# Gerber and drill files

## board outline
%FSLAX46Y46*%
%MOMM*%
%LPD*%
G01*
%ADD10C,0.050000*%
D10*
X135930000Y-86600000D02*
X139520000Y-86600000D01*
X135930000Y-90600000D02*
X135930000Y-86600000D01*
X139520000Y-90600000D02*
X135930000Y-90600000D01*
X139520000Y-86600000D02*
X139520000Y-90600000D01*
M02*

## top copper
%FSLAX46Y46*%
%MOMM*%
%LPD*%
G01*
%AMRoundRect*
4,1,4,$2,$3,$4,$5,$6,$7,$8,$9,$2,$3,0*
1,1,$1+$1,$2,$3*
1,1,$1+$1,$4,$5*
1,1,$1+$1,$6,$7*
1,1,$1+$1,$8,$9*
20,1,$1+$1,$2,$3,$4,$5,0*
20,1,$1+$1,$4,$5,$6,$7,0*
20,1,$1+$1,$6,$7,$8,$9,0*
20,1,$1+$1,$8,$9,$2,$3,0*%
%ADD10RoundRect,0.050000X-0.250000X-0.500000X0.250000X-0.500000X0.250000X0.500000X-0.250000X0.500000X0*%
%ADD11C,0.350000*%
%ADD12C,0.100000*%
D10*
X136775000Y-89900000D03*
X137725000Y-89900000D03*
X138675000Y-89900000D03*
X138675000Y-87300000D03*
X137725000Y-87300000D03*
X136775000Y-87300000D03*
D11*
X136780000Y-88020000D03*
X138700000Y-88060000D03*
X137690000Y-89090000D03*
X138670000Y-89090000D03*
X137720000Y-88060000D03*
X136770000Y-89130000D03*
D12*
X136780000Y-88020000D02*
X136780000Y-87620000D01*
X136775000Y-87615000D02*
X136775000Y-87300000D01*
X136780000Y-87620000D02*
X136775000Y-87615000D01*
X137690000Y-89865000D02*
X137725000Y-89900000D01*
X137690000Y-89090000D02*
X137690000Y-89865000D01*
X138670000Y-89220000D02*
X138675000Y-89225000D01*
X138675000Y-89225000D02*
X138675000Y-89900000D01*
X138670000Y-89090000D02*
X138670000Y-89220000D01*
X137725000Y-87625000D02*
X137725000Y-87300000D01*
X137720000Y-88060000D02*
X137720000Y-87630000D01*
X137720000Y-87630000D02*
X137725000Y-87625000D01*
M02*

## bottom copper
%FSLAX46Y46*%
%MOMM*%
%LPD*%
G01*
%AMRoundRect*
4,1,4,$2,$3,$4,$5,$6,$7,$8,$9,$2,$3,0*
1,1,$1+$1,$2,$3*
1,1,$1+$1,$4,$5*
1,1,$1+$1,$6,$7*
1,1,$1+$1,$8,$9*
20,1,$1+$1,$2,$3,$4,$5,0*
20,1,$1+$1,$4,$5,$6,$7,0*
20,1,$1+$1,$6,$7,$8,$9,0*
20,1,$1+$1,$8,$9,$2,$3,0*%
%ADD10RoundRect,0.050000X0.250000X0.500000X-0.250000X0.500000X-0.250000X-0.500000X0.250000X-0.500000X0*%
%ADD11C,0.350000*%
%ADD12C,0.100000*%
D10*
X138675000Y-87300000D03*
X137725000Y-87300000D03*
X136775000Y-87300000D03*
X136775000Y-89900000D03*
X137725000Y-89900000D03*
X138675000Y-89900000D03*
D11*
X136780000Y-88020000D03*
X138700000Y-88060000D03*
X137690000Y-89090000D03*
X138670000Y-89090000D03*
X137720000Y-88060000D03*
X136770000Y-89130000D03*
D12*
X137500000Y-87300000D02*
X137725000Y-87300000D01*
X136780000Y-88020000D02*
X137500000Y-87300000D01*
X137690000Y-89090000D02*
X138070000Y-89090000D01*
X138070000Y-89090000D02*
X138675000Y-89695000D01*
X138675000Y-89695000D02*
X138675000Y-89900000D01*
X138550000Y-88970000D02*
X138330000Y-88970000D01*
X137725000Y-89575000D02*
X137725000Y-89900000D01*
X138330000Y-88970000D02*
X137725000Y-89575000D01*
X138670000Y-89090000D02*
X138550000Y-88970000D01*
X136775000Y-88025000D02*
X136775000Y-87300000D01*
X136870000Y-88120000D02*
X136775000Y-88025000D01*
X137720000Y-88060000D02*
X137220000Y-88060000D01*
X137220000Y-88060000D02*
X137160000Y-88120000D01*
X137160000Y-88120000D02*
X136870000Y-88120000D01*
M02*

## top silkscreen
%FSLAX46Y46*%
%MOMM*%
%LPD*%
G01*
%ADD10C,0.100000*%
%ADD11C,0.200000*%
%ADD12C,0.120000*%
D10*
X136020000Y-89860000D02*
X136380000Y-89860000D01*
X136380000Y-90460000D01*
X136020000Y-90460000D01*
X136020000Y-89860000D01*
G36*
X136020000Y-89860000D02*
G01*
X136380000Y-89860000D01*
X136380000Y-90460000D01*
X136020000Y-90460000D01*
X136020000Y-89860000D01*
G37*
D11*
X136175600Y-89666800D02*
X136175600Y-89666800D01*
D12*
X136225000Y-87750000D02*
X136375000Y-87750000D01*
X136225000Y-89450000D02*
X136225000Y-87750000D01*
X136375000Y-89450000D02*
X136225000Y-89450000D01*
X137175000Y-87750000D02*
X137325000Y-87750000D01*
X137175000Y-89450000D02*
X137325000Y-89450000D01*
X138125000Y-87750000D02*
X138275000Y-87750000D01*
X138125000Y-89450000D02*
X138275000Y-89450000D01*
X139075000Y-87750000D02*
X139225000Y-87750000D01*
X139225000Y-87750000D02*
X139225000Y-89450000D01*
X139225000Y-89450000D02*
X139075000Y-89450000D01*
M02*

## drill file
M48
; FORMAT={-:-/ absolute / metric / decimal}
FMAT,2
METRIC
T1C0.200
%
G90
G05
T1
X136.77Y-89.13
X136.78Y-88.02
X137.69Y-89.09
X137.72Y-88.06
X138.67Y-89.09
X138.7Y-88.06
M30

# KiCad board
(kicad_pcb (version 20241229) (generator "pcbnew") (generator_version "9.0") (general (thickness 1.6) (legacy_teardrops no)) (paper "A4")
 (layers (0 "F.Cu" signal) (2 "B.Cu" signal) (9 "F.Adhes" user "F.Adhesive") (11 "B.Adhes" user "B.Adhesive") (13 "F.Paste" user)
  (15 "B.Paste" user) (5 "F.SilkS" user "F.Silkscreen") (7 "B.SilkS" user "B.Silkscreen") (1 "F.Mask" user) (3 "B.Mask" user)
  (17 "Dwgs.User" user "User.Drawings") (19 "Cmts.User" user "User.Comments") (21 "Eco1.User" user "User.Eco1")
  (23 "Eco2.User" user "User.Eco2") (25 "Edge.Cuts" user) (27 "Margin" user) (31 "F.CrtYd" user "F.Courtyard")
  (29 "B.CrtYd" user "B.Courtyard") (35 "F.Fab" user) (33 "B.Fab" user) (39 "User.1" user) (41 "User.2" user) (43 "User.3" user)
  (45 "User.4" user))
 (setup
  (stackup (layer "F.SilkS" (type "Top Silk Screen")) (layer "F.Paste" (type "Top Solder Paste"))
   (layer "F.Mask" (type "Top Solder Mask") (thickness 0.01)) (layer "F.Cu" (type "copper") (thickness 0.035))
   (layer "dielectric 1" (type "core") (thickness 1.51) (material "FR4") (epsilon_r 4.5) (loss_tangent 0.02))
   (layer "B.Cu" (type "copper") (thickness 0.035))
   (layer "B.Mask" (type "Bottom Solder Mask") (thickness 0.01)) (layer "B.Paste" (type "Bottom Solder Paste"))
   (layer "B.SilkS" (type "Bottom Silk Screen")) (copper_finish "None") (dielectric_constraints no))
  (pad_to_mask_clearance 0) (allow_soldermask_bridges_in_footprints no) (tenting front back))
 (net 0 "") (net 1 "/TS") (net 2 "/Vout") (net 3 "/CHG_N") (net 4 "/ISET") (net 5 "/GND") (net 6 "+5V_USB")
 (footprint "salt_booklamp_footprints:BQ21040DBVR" (layer "F.Cu") (at 137.725 88.6)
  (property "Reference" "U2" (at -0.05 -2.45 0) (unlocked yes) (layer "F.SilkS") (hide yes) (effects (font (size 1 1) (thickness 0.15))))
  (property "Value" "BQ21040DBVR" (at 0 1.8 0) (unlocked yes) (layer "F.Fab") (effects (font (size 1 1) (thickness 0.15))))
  (fp_line (start -1.5494 1.0668) (end -1.5494 1.0668) (stroke (width 0.2) (type default)) (layer "F.SilkS"))
  (fp_line (start -1.5 -0.85) (end -1.35 -0.85) (stroke (width 0.12) (type default)) (layer "F.SilkS"))
  (fp_line (start -1.5 0.85) (end -1.5 -0.85) (stroke (width 0.12) (type default)) (layer "F.SilkS"))
  (fp_line (start -1.35 0.85) (end -1.5 0.85) (stroke (width 0.12) (type default)) (layer "F.SilkS"))
  (fp_line (start -0.55 -0.85) (end -0.4 -0.85) (stroke (width 0.12) (type default)) (layer "F.SilkS"))
  (fp_line (start -0.55 0.85) (end -0.4 0.85) (stroke (width 0.12) (type default)) (layer "F.SilkS"))
  (fp_line (start 0.4 -0.85) (end 0.55 -0.85) (stroke (width 0.12) (type default)) (layer "F.SilkS"))
  (fp_line (start 0.4 0.85) (end 0.55 0.85) (stroke (width 0.12) (type default)) (layer "F.SilkS"))
  (fp_line (start 1.35 -0.85) (end 1.5 -0.85) (stroke (width 0.12) (type default)) (layer "F.SilkS"))
  (fp_line (start 1.5 -0.85) (end 1.5 0.85) (stroke (width 0.12) (type default)) (layer "F.SilkS"))
  (fp_line (start 1.5 0.85) (end 1.35 0.85) (stroke (width 0.12) (type default)) (layer "F.SilkS"))
  (pad "1" smd roundrect (at -0.95 1.3) (size 0.6 1.1) (layers "F.Cu" "F.Mask" "F.Paste") (roundrect_rratio 0.08333333333) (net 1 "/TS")
   (thermal_bridge_angle 45))
  (pad "2" smd roundrect (at 0 1.3) (size 0.6 1.1) (layers "F.Cu" "F.Mask" "F.Paste") (roundrect_rratio 0.08333333333) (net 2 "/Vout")
   (thermal_bridge_angle 45))
  (pad "3" smd roundrect (at 0.95 1.3) (size 0.6 1.1) (layers "F.Cu" "F.Mask" "F.Paste") (roundrect_rratio 0.08333333333) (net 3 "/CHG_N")
   (thermal_bridge_angle 45))
  (pad "4" smd roundrect (at 0.95 -1.3) (size 0.6 1.1) (layers "F.Cu" "F.Mask" "F.Paste") (roundrect_rratio 0.08333333333) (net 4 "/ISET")
   (thermal_bridge_angle 45))
  (pad "5" smd roundrect (at 0 -1.3) (size 0.6 1.1) (layers "F.Cu" "F.Mask" "F.Paste") (roundrect_rratio 0.08333333333) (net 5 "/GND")
   (thermal_bridge_angle 45))
  (pad "6" smd roundrect (at -0.95 -1.3) (size 0.6 1.1) (layers "F.Cu" "F.Mask" "F.Paste") (roundrect_rratio 0.08333333333)
   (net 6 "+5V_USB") (thermal_bridge_angle 45)))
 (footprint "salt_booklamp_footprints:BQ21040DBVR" (layer "B.Cu") (at 137.725 88.6 180)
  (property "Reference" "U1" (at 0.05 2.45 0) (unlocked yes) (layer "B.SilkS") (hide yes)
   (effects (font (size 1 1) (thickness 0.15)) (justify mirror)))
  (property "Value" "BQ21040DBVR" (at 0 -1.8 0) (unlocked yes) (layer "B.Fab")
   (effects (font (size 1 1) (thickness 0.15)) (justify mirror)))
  (pad "1" smd roundrect (at -0.95 1.3 180) (size 0.6 1.1) (layers "B.Cu" "B.Mask" "B.Paste") (roundrect_rratio 0.08333333333) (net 1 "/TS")
   (thermal_bridge_angle 45))
  (pad "2" smd roundrect (at 0 1.3 180) (size 0.6 1.1) (layers "B.Cu" "B.Mask" "B.Paste") (roundrect_rratio 0.08333333333) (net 6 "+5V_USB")
   (thermal_bridge_angle 45))
  (pad "3" smd roundrect (at 0.95 1.3 180) (size 0.6 1.1) (layers "B.Cu" "B.Mask" "B.Paste") (roundrect_rratio 0.08333333333) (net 5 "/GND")
   (thermal_bridge_angle 45))
  (pad "4" smd roundrect (at 0.95 -1.3 180) (size 0.6 1.1) (layers "B.Cu" "B.Mask" "B.Paste") (roundrect_rratio 0.08333333333)
   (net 4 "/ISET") (thermal_bridge_angle 45))
  (pad "5" smd roundrect (at 0 -1.3 180) (size 0.6 1.1) (layers "B.Cu" "B.Mask" "B.Paste") (roundrect_rratio 0.08333333333) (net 3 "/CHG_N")
   (thermal_bridge_angle 45))
  (pad "6" smd roundrect (at -0.95 -1.3 180) (size 0.6 1.1) (layers "B.Cu" "B.Mask" "B.Paste") (roundrect_rratio 0.08333333333)
   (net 2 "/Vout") (thermal_bridge_angle 45)))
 (gr_rect (start 136.02 89.86) (end 136.38 90.46) (stroke (width 0.1) (type solid)) (fill yes) (layer "F.SilkS"))
 (gr_line (start 135.93 86.6) (end 139.52 86.6) (stroke (width 0.05) (type default)) (layer "Edge.Cuts"))
 (gr_line (start 135.93 90.6) (end 135.93 86.6) (stroke (width 0.05) (type default)) (layer "Edge.Cuts"))
 (gr_line (start 139.52 90.6) (end 135.93 90.6) (stroke (width 0.05) (type default)) (layer "Edge.Cuts"))
 (gr_line (start 139.52 86.6) (end 139.52 90.6) (stroke (width 0.05) (type default)) (layer "Edge.Cuts"))
 (segment (start 136.78 88.02) (end 136.78 87.62) (width 0.1) (layer "F.Cu") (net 6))
 (segment (start 136.775 87.615) (end 136.775 87.3) (width 0.1) (layer "F.Cu") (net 6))
 (segment (start 136.78 87.62) (end 136.775 87.615) (width 0.1) (layer "F.Cu") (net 6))
 (via (at 136.78 88.02) (size 0.35) (drill 0.2) (layers "F.Cu" "B.Cu") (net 6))
 (segment (start 137.5 87.3) (end 137.725 87.3) (width 0.1) (layer "B.Cu") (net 6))
 (segment (start 136.78 88.02) (end 137.5 87.3) (width 0.1) (layer "B.Cu") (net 6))
 (segment (start 137.69 89.865) (end 137.725 89.9) (width 0.1) (layer "F.Cu") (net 2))
 (segment (start 137.69 89.09) (end 137.69 89.865) (width 0.1) (layer "F.Cu") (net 2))
 (via (at 138.7 88.06) (size 0.35) (drill 0.2) (layers "F.Cu" "B.Cu") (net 2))
 (via (at 137.69 89.09) (size 0.35) (drill 0.2) (layers "F.Cu" "B.Cu") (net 2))
 (segment (start 137.69 89.09) (end 138.07 89.09) (width 0.1) (layer "B.Cu") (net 2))
 (segment (start 138.07 89.09) (end 138.675 89.695) (width 0.1) (layer "B.Cu") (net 2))
 (segment (start 138.675 89.695) (end 138.675 89.9) (width 0.1) (layer "B.Cu") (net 2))
 (segment (start 138.67 89.22) (end 138.675 89.225) (width 0.1) (layer "F.Cu") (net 3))
 (segment (start 138.675 89.225) (end 138.675 89.9) (width 0.1) (layer "F.Cu") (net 3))
 (segment (start 138.67 89.09) (end 138.67 89.22) (width 0.1) (layer "F.Cu") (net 3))
 (via (at 138.67 89.09) (size 0.35) (drill 0.2) (layers "F.Cu" "B.Cu") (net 3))
 (segment (start 138.55 88.97) (end 138.33 88.97) (width 0.1) (layer "B.Cu") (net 3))
 (segment (start 137.725 89.575) (end 137.725 89.9) (width 0.1) (layer "B.Cu") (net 3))
 (segment (start 138.33 88.97) (end 137.725 89.575) (width 0.1) (layer "B.Cu") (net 3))
 (segment (start 138.67 89.09) (end 138.55 88.97) (width 0.1) (layer "B.Cu") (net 3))
 (segment (start 137.725 87.625) (end 137.725 87.3) (width 0.1) (layer "F.Cu") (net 5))
 (segment (start 137.72 88.06) (end 137.72 87.63) (width 0.1) (layer "F.Cu") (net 5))
 (segment (start 137.72 87.63) (end 137.725 87.625) (width 0.1) (layer "F.Cu") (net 5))
 (via (at 137.72 88.06) (size 0.35) (drill 0.2) (layers "F.Cu" "B.Cu") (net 5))
 (segment (start 136.775 88.025) (end 136.775 87.3) (width 0.1) (layer "B.Cu") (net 5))
 (segment (start 136.87 88.12) (end 136.775 88.025) (width 0.1) (layer "B.Cu") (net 5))
 (segment (start 137.72 88.06) (end 137.22 88.06) (width 0.1) (layer "B.Cu") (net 5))
 (segment (start 137.22 88.06) (end 137.16 88.12) (width 0.1) (layer "B.Cu") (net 5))
 (segment (start 137.16 88.12) (end 136.87 88.12) (width 0.1) (layer "B.Cu") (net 5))
 (via (at 136.77 89.13) (size 0.35) (drill 0.2) (layers "F.Cu" "B.Cu") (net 1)))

